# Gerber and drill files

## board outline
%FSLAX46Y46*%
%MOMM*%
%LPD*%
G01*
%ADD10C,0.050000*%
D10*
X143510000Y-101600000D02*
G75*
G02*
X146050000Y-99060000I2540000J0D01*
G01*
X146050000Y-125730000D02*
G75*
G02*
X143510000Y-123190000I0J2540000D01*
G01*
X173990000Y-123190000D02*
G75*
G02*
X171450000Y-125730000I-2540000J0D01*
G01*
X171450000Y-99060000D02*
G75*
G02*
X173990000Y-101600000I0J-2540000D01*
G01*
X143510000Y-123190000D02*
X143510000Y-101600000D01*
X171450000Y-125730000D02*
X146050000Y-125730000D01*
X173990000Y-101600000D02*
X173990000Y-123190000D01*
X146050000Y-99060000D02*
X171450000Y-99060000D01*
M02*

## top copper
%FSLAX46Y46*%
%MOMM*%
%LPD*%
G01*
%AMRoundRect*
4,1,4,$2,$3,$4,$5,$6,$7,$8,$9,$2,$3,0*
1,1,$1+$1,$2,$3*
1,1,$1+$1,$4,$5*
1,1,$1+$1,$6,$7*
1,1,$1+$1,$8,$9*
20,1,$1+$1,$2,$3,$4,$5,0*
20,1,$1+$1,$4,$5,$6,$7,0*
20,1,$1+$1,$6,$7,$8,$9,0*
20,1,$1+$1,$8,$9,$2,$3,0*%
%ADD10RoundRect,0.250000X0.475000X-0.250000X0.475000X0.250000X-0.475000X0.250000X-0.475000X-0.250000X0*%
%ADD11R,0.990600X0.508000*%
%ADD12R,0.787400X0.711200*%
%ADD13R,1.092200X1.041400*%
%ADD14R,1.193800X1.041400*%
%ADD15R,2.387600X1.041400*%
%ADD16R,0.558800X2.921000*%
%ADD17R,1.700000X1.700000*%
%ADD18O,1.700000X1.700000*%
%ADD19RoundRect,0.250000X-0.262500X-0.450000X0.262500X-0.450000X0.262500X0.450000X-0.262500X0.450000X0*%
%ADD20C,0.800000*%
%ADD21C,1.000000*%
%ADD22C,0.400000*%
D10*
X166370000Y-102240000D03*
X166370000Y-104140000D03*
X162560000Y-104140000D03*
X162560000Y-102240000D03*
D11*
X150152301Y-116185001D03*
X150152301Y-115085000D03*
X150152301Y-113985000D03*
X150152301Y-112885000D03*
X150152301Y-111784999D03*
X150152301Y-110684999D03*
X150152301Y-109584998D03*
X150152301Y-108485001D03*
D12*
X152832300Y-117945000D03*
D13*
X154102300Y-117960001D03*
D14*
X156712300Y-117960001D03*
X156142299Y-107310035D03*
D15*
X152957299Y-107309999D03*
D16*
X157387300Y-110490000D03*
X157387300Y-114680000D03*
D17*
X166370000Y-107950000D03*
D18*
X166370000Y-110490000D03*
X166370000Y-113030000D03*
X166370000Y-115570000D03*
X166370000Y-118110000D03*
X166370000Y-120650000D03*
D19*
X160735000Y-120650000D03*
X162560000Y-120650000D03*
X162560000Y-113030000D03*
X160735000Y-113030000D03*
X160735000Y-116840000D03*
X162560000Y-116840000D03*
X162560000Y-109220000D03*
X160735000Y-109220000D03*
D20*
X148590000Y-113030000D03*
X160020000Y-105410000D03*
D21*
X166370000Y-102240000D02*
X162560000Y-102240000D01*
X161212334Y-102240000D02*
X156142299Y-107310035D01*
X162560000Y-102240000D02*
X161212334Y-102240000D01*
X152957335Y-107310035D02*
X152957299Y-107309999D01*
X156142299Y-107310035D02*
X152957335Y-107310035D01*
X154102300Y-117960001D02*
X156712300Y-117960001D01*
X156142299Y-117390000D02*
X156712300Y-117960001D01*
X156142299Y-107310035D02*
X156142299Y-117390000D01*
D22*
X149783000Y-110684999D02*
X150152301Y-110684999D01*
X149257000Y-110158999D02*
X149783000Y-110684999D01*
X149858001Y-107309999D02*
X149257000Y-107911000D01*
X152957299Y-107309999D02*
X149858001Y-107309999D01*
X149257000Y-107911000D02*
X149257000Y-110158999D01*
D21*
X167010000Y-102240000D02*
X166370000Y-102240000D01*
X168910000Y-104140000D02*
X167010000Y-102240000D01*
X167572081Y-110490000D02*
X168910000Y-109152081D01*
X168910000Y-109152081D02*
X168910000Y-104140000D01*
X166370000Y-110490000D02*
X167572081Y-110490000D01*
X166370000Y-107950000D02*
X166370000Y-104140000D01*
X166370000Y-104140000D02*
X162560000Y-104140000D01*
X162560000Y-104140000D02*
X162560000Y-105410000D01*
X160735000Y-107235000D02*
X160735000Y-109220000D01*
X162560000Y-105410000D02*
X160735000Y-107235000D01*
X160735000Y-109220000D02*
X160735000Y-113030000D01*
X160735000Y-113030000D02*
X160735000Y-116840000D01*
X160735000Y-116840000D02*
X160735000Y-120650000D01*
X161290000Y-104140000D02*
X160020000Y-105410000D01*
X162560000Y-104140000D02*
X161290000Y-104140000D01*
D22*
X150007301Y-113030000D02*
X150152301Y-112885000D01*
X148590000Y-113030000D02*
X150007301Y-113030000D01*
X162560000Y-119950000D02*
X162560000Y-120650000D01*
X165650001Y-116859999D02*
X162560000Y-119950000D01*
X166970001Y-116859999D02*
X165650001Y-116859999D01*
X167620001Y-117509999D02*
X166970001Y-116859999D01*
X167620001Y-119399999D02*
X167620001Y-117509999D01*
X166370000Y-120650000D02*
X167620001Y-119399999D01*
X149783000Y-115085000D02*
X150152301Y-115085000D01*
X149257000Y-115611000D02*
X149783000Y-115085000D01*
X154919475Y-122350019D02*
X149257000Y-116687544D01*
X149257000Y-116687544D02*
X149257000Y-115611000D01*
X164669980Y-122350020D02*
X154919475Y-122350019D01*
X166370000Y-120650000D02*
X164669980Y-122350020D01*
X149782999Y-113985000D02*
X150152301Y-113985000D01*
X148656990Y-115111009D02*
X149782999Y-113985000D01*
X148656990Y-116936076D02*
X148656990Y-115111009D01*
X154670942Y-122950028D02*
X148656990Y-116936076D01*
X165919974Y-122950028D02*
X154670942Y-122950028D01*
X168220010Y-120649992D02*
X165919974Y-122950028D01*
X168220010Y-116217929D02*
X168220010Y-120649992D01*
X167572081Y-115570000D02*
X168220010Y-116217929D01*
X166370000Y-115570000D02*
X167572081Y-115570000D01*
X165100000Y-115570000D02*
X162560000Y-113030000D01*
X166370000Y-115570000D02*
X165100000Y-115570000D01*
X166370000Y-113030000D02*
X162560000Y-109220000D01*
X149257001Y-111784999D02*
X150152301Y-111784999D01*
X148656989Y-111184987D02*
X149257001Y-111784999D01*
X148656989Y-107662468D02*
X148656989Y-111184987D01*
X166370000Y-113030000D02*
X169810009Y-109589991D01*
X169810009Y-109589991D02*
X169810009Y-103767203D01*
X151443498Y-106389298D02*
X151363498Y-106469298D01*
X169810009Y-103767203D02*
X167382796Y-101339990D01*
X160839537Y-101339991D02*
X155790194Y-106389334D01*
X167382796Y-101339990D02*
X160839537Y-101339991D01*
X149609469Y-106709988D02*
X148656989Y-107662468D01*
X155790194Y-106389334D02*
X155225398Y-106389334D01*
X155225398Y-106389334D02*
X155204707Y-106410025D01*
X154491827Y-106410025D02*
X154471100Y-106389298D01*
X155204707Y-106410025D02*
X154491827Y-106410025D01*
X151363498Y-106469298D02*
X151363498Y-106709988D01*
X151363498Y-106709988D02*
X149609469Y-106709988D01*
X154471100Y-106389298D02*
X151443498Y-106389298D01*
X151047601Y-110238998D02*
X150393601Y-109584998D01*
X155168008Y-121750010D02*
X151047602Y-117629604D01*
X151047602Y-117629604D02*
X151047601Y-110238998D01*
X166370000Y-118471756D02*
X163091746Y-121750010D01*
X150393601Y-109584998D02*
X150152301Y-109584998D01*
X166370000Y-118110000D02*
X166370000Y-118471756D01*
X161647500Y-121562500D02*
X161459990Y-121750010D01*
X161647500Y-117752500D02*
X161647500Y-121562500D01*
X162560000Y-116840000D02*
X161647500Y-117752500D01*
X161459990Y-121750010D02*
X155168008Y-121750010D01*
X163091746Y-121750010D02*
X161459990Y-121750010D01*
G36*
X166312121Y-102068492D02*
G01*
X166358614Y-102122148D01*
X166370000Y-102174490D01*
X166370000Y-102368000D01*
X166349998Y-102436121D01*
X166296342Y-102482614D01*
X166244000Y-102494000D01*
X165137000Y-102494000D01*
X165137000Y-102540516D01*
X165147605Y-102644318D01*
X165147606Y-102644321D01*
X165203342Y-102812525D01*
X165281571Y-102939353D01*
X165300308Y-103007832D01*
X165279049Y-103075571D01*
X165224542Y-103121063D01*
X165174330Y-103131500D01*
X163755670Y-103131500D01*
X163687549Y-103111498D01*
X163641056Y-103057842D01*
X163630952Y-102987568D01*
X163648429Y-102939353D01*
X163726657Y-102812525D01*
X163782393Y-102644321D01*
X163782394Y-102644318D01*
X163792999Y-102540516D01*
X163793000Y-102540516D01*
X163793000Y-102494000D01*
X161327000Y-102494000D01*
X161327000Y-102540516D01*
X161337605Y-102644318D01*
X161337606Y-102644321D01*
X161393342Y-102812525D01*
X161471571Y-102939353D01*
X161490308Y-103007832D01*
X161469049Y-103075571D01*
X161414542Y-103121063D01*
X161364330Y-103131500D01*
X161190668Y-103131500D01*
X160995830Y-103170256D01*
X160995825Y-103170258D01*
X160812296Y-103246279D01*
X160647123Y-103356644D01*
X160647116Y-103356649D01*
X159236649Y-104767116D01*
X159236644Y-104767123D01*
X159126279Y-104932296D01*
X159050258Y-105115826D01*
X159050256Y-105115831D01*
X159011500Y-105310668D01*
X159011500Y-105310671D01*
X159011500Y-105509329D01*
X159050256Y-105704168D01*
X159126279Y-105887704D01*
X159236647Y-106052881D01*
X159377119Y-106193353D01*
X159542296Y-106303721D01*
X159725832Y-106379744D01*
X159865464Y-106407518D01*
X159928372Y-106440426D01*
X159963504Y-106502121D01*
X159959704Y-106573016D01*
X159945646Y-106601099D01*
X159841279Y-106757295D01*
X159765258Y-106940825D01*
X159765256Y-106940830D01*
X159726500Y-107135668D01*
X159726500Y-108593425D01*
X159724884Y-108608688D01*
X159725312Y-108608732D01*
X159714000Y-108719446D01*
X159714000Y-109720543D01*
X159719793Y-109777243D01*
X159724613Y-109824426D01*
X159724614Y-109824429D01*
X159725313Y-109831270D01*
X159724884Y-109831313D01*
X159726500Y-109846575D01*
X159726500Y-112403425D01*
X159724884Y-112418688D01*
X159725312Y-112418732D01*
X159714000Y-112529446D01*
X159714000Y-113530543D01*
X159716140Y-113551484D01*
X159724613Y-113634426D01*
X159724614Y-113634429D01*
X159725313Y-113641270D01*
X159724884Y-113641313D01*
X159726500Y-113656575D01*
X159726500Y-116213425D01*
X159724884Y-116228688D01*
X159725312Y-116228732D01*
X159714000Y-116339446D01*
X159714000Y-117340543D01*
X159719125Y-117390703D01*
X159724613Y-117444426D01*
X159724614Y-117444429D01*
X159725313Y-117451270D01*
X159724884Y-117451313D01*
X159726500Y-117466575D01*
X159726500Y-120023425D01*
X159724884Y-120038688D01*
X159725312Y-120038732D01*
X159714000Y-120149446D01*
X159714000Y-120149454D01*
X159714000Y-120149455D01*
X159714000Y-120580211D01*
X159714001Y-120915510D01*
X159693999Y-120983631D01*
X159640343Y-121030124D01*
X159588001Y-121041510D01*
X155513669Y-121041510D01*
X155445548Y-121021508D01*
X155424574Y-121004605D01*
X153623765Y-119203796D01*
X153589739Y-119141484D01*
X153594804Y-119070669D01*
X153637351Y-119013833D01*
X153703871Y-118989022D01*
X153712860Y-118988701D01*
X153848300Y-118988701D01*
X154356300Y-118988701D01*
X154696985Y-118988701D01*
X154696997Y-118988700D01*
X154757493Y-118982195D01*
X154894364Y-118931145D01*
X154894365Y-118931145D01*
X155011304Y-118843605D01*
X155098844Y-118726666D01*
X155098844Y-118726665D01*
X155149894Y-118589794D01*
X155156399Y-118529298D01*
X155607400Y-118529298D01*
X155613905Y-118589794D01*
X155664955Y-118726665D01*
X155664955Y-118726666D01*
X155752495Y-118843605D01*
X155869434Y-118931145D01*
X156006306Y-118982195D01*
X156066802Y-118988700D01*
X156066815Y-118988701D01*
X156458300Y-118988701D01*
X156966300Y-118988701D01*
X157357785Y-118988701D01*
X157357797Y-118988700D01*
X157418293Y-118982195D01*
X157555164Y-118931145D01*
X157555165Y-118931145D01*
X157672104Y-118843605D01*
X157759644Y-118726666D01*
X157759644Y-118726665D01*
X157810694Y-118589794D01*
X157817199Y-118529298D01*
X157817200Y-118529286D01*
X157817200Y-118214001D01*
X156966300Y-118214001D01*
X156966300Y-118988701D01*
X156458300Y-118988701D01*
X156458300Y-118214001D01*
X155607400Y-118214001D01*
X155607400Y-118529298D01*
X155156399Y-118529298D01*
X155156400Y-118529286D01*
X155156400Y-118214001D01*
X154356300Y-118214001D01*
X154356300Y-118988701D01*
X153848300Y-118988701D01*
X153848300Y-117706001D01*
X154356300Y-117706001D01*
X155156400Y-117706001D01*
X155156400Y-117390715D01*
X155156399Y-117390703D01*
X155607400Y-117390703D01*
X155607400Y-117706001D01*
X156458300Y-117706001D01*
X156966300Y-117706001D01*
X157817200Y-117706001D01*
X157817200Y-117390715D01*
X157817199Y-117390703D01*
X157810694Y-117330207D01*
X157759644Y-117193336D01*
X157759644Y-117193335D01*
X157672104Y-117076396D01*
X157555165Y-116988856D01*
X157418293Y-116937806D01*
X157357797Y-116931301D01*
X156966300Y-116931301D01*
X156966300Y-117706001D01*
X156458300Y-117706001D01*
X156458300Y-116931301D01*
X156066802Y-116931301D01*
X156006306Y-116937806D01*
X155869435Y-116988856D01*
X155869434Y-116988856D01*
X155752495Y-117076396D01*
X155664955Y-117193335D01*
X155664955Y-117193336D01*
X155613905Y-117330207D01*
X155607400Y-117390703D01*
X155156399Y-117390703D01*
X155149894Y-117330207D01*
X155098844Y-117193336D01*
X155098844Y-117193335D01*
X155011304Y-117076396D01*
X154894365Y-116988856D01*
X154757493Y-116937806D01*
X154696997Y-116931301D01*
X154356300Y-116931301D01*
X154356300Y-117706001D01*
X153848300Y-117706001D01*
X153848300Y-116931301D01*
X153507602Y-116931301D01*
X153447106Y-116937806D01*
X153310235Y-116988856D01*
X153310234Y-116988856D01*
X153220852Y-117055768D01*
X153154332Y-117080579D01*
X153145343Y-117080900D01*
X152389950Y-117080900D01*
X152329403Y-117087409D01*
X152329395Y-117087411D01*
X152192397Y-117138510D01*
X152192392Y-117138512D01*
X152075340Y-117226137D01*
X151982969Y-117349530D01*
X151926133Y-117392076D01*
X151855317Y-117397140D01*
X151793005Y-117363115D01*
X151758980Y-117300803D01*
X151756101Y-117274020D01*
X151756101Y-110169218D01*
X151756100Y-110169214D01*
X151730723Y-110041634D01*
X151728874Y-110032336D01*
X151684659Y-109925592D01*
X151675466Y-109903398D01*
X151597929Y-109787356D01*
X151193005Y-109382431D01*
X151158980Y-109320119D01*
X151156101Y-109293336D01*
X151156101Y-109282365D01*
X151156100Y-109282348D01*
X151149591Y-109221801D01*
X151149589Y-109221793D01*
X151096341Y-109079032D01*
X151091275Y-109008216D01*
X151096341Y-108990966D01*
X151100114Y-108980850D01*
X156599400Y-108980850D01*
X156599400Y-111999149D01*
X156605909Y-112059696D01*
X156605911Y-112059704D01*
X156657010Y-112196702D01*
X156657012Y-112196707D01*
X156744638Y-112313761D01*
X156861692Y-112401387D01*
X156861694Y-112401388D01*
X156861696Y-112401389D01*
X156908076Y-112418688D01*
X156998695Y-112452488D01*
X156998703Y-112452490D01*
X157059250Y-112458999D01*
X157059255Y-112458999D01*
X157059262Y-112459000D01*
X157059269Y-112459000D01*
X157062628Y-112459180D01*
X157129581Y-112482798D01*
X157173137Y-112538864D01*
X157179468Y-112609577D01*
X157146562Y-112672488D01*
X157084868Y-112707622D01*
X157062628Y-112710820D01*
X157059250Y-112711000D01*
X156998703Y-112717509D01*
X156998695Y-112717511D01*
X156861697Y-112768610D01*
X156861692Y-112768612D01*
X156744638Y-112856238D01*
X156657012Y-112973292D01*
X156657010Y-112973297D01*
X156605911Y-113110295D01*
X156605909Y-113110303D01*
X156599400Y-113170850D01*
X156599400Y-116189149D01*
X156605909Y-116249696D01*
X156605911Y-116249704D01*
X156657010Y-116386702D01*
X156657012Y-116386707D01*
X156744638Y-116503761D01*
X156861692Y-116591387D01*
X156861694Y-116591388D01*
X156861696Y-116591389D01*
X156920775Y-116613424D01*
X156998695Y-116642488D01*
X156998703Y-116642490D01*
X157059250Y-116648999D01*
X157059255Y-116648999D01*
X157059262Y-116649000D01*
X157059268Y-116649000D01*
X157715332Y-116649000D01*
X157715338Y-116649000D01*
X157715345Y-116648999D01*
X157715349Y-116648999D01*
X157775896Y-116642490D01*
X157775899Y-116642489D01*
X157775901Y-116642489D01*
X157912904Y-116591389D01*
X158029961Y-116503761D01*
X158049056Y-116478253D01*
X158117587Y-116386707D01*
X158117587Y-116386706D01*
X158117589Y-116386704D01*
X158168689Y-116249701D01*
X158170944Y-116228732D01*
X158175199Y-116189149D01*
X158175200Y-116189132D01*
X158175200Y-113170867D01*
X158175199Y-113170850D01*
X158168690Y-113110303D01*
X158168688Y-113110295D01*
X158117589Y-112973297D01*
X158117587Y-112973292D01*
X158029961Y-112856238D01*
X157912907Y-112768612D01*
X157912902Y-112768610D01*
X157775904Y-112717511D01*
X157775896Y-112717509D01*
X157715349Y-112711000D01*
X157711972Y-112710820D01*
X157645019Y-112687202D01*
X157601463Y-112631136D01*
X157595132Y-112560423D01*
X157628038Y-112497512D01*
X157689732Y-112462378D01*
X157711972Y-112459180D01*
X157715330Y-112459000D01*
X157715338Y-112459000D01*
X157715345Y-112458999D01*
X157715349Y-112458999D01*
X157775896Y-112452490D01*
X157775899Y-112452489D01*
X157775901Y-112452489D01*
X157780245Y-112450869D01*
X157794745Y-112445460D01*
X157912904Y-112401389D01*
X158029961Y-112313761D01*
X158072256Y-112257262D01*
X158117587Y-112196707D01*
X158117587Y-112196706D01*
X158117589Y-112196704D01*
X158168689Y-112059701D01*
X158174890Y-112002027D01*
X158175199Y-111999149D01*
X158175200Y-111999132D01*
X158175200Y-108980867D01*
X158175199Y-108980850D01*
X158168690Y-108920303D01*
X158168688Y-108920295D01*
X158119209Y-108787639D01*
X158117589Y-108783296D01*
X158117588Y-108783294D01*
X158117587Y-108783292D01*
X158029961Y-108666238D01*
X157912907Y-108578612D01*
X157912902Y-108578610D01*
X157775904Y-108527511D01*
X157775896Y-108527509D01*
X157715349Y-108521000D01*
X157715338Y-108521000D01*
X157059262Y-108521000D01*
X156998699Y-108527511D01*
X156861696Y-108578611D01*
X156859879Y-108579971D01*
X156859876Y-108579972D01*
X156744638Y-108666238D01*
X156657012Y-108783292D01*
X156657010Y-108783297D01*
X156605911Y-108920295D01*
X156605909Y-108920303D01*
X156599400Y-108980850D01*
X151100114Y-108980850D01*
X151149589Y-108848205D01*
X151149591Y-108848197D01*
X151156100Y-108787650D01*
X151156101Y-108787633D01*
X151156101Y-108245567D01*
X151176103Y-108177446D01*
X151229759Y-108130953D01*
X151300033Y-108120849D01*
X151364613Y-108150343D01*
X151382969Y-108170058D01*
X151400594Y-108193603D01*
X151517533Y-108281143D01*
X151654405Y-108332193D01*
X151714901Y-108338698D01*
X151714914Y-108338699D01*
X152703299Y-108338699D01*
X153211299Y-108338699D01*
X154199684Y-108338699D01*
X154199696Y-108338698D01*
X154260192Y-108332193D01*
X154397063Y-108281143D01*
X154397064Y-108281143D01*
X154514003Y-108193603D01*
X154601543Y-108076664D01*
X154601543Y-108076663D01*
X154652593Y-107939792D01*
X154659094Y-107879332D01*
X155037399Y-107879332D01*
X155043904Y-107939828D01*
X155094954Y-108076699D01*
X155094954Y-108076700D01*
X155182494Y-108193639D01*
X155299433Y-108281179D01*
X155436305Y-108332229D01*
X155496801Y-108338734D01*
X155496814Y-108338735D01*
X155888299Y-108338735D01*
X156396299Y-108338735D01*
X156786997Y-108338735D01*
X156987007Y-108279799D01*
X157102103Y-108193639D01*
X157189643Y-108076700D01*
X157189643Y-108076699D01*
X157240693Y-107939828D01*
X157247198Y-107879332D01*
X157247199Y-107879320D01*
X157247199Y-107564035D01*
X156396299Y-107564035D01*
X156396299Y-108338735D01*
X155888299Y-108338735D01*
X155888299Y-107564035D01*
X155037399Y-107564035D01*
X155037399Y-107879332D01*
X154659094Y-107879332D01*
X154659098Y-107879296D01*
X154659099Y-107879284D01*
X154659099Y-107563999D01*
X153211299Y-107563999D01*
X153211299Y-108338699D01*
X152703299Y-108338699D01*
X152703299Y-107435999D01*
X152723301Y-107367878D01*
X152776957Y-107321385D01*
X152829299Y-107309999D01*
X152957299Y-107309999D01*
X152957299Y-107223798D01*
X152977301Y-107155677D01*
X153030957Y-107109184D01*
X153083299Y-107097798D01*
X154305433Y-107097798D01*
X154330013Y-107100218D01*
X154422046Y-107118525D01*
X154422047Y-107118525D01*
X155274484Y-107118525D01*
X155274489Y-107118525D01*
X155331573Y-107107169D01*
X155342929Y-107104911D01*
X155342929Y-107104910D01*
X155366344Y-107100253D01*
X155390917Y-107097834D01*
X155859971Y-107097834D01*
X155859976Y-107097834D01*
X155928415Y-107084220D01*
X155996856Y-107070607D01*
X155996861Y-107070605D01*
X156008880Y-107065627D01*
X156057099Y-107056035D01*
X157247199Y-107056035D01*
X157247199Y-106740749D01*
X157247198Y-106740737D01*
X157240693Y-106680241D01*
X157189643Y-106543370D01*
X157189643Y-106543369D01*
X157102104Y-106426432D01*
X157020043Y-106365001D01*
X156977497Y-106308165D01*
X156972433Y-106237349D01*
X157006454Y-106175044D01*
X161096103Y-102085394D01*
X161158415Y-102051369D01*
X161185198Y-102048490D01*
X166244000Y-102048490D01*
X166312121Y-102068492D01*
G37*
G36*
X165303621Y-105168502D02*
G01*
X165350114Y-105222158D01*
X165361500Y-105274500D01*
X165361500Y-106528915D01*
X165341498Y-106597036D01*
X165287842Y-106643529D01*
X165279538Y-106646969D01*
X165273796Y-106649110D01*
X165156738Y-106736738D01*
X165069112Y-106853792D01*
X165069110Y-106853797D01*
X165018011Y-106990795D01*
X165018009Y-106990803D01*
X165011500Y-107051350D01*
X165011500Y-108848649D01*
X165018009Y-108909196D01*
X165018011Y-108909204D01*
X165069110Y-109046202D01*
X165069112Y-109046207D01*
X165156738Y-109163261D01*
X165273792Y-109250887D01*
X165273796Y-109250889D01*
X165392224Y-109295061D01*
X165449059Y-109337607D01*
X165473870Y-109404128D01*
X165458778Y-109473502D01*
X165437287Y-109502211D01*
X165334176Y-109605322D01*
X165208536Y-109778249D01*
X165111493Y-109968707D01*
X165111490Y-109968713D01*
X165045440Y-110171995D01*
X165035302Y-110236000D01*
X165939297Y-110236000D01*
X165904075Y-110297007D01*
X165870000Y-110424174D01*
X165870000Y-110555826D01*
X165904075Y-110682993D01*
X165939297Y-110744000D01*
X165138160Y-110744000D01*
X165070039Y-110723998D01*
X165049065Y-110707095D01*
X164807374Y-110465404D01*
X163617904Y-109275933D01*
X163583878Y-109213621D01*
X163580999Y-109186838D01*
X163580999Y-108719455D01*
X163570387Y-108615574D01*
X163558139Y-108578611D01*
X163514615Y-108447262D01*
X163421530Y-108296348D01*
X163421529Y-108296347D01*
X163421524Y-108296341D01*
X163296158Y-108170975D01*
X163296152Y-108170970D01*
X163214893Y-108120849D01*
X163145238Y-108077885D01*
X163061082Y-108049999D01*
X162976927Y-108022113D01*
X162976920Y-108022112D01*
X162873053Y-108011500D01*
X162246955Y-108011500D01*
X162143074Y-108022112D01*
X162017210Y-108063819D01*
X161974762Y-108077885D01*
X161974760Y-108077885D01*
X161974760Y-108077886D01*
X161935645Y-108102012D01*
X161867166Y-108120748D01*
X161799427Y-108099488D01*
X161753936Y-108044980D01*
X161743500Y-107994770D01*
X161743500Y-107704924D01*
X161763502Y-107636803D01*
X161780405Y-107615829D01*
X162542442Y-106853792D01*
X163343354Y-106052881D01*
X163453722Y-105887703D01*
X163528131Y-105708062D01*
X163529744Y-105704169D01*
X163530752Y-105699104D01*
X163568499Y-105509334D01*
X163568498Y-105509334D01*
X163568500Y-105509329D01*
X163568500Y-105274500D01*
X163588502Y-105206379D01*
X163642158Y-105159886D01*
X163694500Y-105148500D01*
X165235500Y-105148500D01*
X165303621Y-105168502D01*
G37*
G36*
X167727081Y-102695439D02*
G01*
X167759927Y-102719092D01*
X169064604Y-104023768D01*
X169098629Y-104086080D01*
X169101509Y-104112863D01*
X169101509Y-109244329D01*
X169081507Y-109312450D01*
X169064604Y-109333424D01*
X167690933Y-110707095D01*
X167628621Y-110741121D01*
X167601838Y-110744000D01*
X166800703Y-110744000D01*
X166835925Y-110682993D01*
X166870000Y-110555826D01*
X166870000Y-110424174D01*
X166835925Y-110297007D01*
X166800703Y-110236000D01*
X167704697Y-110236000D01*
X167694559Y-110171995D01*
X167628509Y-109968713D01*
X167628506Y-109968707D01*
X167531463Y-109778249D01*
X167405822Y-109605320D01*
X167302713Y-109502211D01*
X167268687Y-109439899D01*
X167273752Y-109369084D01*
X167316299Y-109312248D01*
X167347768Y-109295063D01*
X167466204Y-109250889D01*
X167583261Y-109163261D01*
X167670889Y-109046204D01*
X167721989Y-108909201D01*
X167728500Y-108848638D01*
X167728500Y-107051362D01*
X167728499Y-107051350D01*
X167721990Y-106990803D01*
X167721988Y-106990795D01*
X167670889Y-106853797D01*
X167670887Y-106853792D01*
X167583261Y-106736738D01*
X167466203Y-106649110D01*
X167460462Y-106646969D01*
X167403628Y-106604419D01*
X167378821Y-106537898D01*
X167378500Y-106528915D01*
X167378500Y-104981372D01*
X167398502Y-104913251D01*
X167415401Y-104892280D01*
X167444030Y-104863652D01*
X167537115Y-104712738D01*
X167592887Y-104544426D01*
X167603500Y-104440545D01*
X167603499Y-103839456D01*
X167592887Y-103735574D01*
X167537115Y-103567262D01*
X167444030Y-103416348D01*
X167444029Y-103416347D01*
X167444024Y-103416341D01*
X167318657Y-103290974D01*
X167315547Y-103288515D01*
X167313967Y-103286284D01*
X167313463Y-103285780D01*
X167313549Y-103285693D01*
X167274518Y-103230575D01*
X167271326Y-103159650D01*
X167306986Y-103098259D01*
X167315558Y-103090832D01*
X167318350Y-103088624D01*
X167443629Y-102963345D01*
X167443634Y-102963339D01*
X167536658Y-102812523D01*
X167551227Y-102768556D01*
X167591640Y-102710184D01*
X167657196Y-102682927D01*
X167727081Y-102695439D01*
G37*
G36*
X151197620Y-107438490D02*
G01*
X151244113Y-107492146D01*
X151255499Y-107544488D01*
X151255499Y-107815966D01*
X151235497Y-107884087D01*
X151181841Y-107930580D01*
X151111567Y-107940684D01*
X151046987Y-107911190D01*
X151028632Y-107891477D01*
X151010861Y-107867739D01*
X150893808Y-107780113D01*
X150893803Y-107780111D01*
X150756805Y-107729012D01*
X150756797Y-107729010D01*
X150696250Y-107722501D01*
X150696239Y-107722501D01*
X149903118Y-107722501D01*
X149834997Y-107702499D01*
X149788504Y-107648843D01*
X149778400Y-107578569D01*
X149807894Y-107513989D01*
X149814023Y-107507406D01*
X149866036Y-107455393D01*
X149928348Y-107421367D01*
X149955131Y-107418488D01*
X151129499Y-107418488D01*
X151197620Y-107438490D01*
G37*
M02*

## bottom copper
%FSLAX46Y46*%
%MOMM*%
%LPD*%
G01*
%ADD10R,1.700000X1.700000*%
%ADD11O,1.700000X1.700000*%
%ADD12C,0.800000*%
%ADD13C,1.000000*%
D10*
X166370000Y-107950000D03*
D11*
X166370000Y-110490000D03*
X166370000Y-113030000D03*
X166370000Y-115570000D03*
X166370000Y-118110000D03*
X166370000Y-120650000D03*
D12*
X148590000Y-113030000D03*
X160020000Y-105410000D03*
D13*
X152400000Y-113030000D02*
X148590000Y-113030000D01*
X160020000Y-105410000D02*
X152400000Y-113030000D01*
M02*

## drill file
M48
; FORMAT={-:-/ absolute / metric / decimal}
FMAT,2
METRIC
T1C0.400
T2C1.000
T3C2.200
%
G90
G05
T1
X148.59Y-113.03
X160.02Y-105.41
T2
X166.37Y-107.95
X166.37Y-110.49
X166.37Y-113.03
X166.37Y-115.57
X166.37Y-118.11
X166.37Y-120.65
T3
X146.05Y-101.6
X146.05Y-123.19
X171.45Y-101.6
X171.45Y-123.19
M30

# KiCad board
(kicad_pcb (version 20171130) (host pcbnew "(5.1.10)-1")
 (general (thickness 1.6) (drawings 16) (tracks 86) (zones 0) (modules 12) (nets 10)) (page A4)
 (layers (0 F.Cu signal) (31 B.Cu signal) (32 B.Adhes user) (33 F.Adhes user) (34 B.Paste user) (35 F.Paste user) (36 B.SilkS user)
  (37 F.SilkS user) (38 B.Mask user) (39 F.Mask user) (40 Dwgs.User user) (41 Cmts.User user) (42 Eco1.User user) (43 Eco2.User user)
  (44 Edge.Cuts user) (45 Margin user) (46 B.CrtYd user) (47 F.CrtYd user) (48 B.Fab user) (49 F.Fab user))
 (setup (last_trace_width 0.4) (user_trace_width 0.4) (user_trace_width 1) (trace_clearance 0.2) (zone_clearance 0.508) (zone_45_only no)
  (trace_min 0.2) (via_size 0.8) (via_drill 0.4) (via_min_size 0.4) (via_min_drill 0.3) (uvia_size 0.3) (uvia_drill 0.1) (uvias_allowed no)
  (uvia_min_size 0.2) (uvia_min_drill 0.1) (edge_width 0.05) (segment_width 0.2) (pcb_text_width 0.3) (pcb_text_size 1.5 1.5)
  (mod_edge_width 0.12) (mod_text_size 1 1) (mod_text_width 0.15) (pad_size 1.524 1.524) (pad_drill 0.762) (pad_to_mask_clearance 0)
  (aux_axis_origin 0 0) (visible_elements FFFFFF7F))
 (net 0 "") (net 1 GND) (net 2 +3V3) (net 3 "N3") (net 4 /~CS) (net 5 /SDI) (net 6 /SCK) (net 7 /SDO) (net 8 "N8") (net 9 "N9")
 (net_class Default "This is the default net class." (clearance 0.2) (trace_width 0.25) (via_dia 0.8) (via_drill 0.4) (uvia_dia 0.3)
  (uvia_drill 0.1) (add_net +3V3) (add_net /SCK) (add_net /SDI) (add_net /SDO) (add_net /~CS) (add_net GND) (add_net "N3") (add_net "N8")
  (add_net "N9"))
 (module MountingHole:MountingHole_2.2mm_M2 (layer F.Cu) (at 171.45 123.19)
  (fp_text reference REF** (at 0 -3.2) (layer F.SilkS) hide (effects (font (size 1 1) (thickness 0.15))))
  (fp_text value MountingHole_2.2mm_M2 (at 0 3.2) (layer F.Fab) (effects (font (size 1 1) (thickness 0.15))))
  (pad 1 np_thru_hole circle (at 0 0) (size 2.2 2.2) (drill 2.2) (layers *.Cu *.Mask)))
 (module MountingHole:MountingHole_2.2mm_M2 (layer F.Cu) (at 146.05 123.19)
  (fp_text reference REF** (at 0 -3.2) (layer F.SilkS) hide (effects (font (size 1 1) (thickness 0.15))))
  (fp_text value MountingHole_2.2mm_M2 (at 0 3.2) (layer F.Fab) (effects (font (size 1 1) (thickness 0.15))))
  (pad 1 np_thru_hole circle (at 0 0) (size 2.2 2.2) (drill 2.2) (layers *.Cu *.Mask)))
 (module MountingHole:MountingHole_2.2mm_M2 (layer F.Cu) (at 146.05 101.6)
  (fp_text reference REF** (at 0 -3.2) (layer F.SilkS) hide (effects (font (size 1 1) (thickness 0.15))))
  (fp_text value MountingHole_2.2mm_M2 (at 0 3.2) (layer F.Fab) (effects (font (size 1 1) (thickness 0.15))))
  (pad 1 np_thru_hole circle (at 0 0) (size 2.2 2.2) (drill 2.2) (layers *.Cu *.Mask)))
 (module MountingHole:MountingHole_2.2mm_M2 (layer F.Cu) (at 171.45 101.6)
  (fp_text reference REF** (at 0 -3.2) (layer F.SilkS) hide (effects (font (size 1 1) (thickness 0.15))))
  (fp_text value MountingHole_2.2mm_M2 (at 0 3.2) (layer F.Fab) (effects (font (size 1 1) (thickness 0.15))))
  (pad 1 np_thru_hole circle (at 0 0) (size 2.2 2.2) (drill 2.2) (layers *.Cu *.Mask)))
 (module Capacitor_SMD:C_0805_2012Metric (layer F.Cu) (at 166.37 103.19 90)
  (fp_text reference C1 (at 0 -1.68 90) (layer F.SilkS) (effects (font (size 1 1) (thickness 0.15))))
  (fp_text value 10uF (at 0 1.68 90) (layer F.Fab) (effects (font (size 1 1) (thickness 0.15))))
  (pad 2 smd roundrect (at 0.95 0 90) (size 1 1.45) (layers F.Cu F.Paste F.Mask) (roundrect_rratio 0.25) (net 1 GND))
  (pad 1 smd roundrect (at -0.95 0 90) (size 1 1.45) (layers F.Cu F.Paste F.Mask) (roundrect_rratio 0.25) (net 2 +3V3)))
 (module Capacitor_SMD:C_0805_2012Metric (layer F.Cu) (at 162.56 103.19 90)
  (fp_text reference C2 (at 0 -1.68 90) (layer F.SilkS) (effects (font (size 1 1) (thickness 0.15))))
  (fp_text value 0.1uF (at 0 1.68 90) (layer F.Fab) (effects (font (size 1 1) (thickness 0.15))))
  (pad 1 smd roundrect (at -0.95 0 90) (size 1 1.45) (layers F.Cu F.Paste F.Mask) (roundrect_rratio 0.25) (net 2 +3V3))
  (pad 2 smd roundrect (at 0.95 0 90) (size 1 1.45) (layers F.Cu F.Paste F.Mask) (roundrect_rratio 0.25) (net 1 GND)))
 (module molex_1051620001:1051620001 (layer F.Cu) (at 153.67 112.635 270)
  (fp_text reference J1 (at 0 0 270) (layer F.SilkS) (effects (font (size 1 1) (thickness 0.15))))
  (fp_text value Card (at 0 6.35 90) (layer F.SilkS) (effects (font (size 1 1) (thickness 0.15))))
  (pad P1 smd rect (at 3.550001 3.517699 270) (size 0.508 0.9906) (layers F.Cu F.Paste F.Mask) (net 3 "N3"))
  (pad P2 smd rect (at 2.45 3.517699 270) (size 0.508 0.9906) (layers F.Cu F.Paste F.Mask) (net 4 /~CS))
  (pad P3 smd rect (at 1.35 3.517699 270) (size 0.508 0.9906) (layers F.Cu F.Paste F.Mask) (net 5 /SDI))
  (pad P4 smd rect (at 0.25 3.517699 270) (size 0.508 0.9906) (layers F.Cu F.Paste F.Mask) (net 2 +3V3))
  (pad P5 smd rect (at -0.850001 3.517699 270) (size 0.508 0.9906) (layers F.Cu F.Paste F.Mask) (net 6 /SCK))
  (pad P6 smd rect (at -1.950001 3.517699 270) (size 0.508 0.9906) (layers F.Cu F.Paste F.Mask) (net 1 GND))
  (pad P7 smd rect (at -3.050002 3.517699 270) (size 0.508 0.9906) (layers F.Cu F.Paste F.Mask) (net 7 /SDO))
  (pad P8 smd rect (at -4.149999 3.517699 270) (size 0.508 0.9906) (layers F.Cu F.Paste F.Mask) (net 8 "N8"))
  (pad P9 smd rect (at 5.31 0.8377 270) (size 0.7112 0.7874) (layers F.Cu F.Paste F.Mask) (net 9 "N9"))
  (pad G1 smd rect (at 5.325001 -0.4323 270) (size 1.0414 1.0922) (layers F.Cu F.Paste F.Mask) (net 1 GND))
  (pad G2 smd rect (at 5.325001 -3.0423 270) (size 1.0414 1.1938) (layers F.Cu F.Paste F.Mask) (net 1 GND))
  (pad G3 smd rect (at -5.324965 -2.472299 270) (size 1.0414 1.1938) (layers F.Cu F.Paste F.Mask) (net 1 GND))
  (pad G4 smd rect (at -5.325001 0.712701 270) (size 1.0414 2.3876) (layers F.Cu F.Paste F.Mask) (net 1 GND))
  (pad 14 smd rect (at -2.145 -3.7173 270) (size 2.921 0.5588) (layers F.Cu F.Paste F.Mask))
  (pad 15 smd rect (at 2.045 -3.7173 270) (size 2.921 0.5588) (layers F.Cu F.Paste F.Mask)))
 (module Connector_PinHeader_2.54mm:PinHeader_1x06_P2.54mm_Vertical (layer F.Cu) (at 166.37 107.95)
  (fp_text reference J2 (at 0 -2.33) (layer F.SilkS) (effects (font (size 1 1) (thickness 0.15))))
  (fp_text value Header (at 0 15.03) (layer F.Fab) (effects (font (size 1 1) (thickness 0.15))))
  (pad 1 thru_hole rect (at 0 0) (size 1.7 1.7) (drill 1) (layers *.Cu *.Mask) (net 2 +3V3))
  (pad 2 thru_hole oval (at 0 2.54) (size 1.7 1.7) (drill 1) (layers *.Cu *.Mask) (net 1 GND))
  (pad 3 thru_hole oval (at 0 5.08) (size 1.7 1.7) (drill 1) (layers *.Cu *.Mask) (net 6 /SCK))
  (pad 4 thru_hole oval (at 0 7.62) (size 1.7 1.7) (drill 1) (layers *.Cu *.Mask) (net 5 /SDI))
  (pad 5 thru_hole oval (at 0 10.16) (size 1.7 1.7) (drill 1) (layers *.Cu *.Mask) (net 7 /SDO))
  (pad 6 thru_hole oval (at 0 12.7) (size 1.7 1.7) (drill 1) (layers *.Cu *.Mask) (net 4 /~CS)))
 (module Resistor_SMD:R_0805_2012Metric (layer F.Cu) (at 161.6475 120.65)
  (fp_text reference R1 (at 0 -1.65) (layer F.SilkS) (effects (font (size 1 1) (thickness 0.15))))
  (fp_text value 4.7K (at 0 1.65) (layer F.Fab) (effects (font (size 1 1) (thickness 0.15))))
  (pad 1 smd roundrect (at -0.9125 0) (size 1.025 1.4) (layers F.Cu F.Paste F.Mask) (roundrect_rratio 0.243902) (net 2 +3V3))
  (pad 2 smd roundrect (at 0.9125 0) (size 1.025 1.4) (layers F.Cu F.Paste F.Mask) (roundrect_rratio 0.243902) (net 4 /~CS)))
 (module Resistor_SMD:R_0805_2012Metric (layer F.Cu) (at 161.6475 113.03)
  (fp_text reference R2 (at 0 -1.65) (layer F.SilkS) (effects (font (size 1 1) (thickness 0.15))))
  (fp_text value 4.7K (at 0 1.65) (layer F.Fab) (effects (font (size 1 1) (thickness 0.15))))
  (pad 2 smd roundrect (at 0.9125 0) (size 1.025 1.4) (layers F.Cu F.Paste F.Mask) (roundrect_rratio 0.243902) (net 5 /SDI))
  (pad 1 smd roundrect (at -0.9125 0) (size 1.025 1.4) (layers F.Cu F.Paste F.Mask) (roundrect_rratio 0.243902) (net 2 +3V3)))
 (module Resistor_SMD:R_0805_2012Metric (layer F.Cu) (at 161.6475 116.84)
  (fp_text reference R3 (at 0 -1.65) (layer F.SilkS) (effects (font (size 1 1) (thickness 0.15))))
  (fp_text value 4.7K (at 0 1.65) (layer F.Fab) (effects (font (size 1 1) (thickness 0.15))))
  (pad 1 smd roundrect (at -0.9125 0) (size 1.025 1.4) (layers F.Cu F.Paste F.Mask) (roundrect_rratio 0.243902) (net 2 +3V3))
  (pad 2 smd roundrect (at 0.9125 0) (size 1.025 1.4) (layers F.Cu F.Paste F.Mask) (roundrect_rratio 0.243902) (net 7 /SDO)))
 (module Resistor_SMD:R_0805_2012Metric (layer F.Cu) (at 161.6475 109.22)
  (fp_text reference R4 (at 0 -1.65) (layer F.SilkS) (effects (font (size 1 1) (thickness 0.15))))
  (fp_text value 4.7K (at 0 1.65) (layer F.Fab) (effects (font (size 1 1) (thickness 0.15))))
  (pad 2 smd roundrect (at 0.9125 0) (size 1.025 1.4) (layers F.Cu F.Paste F.Mask) (roundrect_rratio 0.243902) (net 6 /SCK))
  (pad 1 smd roundrect (at -0.9125 0) (size 1.025 1.4) (layers F.Cu F.Paste F.Mask) (roundrect_rratio 0.243902) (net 2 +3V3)))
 (gr_arc (start 146.05 101.6) (end 146.05 99.06) (angle -90) (layer Edge.Cuts) (width 0.05))
 (gr_arc (start 146.05 123.19) (end 143.51 123.19) (angle -90) (layer Edge.Cuts) (width 0.05))
 (gr_arc (start 171.45 123.19) (end 171.45 125.73) (angle -90) (layer Edge.Cuts) (width 0.05))
 (gr_arc (start 171.45 101.6) (end 173.99 101.6) (angle -90) (layer Edge.Cuts) (width 0.05))
 (gr_line (start 143.51 123.19) (end 143.51 101.6) (layer Edge.Cuts) (width 0.05))
 (gr_line (start 171.45 125.73) (end 146.05 125.73) (layer Edge.Cuts) (width 0.05))
 (gr_line (start 173.99 101.6) (end 173.99 123.19) (layer Edge.Cuts) (width 0.05))
 (gr_line (start 146.05 99.06) (end 171.45 99.06) (layer Edge.Cuts) (width 0.05))
 (segment (start 166.37 102.24) (end 162.56 102.24) (width 1) (layer F.Cu) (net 1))
 (segment (start 161.212334 102.24) (end 156.142299 107.310035) (width 1) (layer F.Cu) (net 1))
 (segment (start 162.56 102.24) (end 161.212334 102.24) (width 1) (layer F.Cu) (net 1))
 (segment (start 152.957335 107.310035) (end 152.957299 107.309999) (width 1) (layer F.Cu) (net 1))
 (segment (start 156.142299 107.310035) (end 152.957335 107.310035) (width 1) (layer F.Cu) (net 1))
 (segment (start 154.1023 117.960001) (end 156.7123 117.960001) (width 1) (layer F.Cu) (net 1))
 (segment (start 156.142299 117.39) (end 156.7123 117.960001) (width 1) (layer F.Cu) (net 1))
 (segment (start 156.142299 107.310035) (end 156.142299 117.39) (width 1) (layer F.Cu) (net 1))
 (segment (start 149.783 110.684999) (end 150.152301 110.684999) (width 0.4) (layer F.Cu) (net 1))
 (segment (start 149.257 110.158999) (end 149.783 110.684999) (width 0.4) (layer F.Cu) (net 1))
 (segment (start 149.858001 107.309999) (end 149.257 107.911) (width 0.4) (layer F.Cu) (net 1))
 (segment (start 152.957299 107.309999) (end 149.858001 107.309999) (width 0.4) (layer F.Cu) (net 1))
 (segment (start 149.257 107.911) (end 149.257 110.158999) (width 0.4) (layer F.Cu) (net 1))
 (segment (start 167.01 102.24) (end 166.37 102.24) (width 1) (layer F.Cu) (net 1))
 (segment (start 168.91 104.14) (end 167.01 102.24) (width 1) (layer F.Cu) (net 1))
 (segment (start 167.572081 110.49) (end 168.91 109.152081) (width 1) (layer F.Cu) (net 1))
 (segment (start 168.91 109.152081) (end 168.91 104.14) (width 1) (layer F.Cu) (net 1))
 (segment (start 166.37 110.49) (end 167.572081 110.49) (width 1) (layer F.Cu) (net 1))
 (segment (start 166.37 107.95) (end 166.37 104.14) (width 1) (layer F.Cu) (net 2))
 (segment (start 166.37 104.14) (end 162.56 104.14) (width 1) (layer F.Cu) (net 2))
 (segment (start 162.56 104.14) (end 162.56 105.41) (width 1) (layer F.Cu) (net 2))
 (segment (start 160.735 107.235) (end 160.735 109.22) (width 1) (layer F.Cu) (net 2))
 (segment (start 162.56 105.41) (end 160.735 107.235) (width 1) (layer F.Cu) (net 2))
 (segment (start 160.735 109.22) (end 160.735 113.03) (width 1) (layer F.Cu) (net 2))
 (segment (start 160.735 113.03) (end 160.735 116.84) (width 1) (layer F.Cu) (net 2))
 (segment (start 160.735 116.84) (end 160.735 120.65) (width 1) (layer F.Cu) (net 2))
 (via (at 148.59 113.03) (size 0.8) (drill 0.4) (layers F.Cu B.Cu) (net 2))
 (via (at 160.02 105.41) (size 0.8) (drill 0.4) (layers F.Cu B.Cu) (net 2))
 (segment (start 161.29 104.14) (end 160.02 105.41) (width 1) (layer F.Cu) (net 2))
 (segment (start 162.56 104.14) (end 161.29 104.14) (width 1) (layer F.Cu) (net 2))
 (segment (start 152.4 113.03) (end 148.59 113.03) (width 1) (layer B.Cu) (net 2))
 (segment (start 160.02 105.41) (end 152.4 113.03) (width 1) (layer B.Cu) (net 2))
 (segment (start 150.007301 113.03) (end 150.152301 112.885) (width 0.4) (layer F.Cu) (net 2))
 (segment (start 148.59 113.03) (end 150.007301 113.03) (width 0.4) (layer F.Cu) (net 2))
 (segment (start 162.56 119.95) (end 162.56 120.65) (width 0.4) (layer F.Cu) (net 4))
 (segment (start 165.650001 116.859999) (end 162.56 119.95) (width 0.4) (layer F.Cu) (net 4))
 (segment (start 166.970001 116.859999) (end 165.650001 116.859999) (width 0.4) (layer F.Cu) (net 4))
 (segment (start 167.620001 117.509999) (end 166.970001 116.859999) (width 0.4) (layer F.Cu) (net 4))
 (segment (start 167.620001 119.399999) (end 167.620001 117.509999) (width 0.4) (layer F.Cu) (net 4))
 (segment (start 166.37 120.65) (end 167.620001 119.399999) (width 0.4) (layer F.Cu) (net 4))
 (segment (start 149.783 115.085) (end 150.152301 115.085) (width 0.4) (layer F.Cu) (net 4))
 (segment (start 149.257 115.611) (end 149.783 115.085) (width 0.4) (layer F.Cu) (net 4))
 (segment (start 154.919475 122.350019) (end 149.257 116.687544) (width 0.4) (layer F.Cu) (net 4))
 (segment (start 149.257 116.687544) (end 149.257 115.611) (width 0.4) (layer F.Cu) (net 4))
 (segment (start 164.66998 122.35002) (end 154.919475 122.350019) (width 0.4) (layer F.Cu) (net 4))
 (segment (start 166.37 120.65) (end 164.66998 122.35002) (width 0.4) (layer F.Cu) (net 4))
 (segment (start 149.782999 113.985) (end 150.152301 113.985) (width 0.4) (layer F.Cu) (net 5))
 (segment (start 148.65699 115.111009) (end 149.782999 113.985) (width 0.4) (layer F.Cu) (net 5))
 (segment (start 148.65699 116.936076) (end 148.65699 115.111009) (width 0.4) (layer F.Cu) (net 5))
 (segment (start 154.670942 122.950028) (end 148.65699 116.936076) (width 0.4) (layer F.Cu) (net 5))
 (segment (start 165.919974 122.950028) (end 154.670942 122.950028) (width 0.4) (layer F.Cu) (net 5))
 (segment (start 168.22001 120.649992) (end 165.919974 122.950028) (width 0.4) (layer F.Cu) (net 5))
 (segment (start 168.22001 116.217929) (end 168.22001 120.649992) (width 0.4) (layer F.Cu) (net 5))
 (segment (start 167.572081 115.57) (end 168.22001 116.217929) (width 0.4) (layer F.Cu) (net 5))
 (segment (start 166.37 115.57) (end 167.572081 115.57) (width 0.4) (layer F.Cu) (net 5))
 (segment (start 165.1 115.57) (end 162.56 113.03) (width 0.4) (layer F.Cu) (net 5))
 (segment (start 166.37 115.57) (end 165.1 115.57) (width 0.4) (layer F.Cu) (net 5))
 (segment (start 166.37 113.03) (end 162.56 109.22) (width 0.4) (layer F.Cu) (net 6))
 (segment (start 149.257001 111.784999) (end 150.152301 111.784999) (width 0.4) (layer F.Cu) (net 6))
 (segment (start 148.656989 111.184987) (end 149.257001 111.784999) (width 0.4) (layer F.Cu) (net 6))
 (segment (start 148.656989 107.662468) (end 148.656989 111.184987) (width 0.4) (layer F.Cu) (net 6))
 (segment (start 166.37 113.03) (end 169.810009 109.589991) (width 0.4) (layer F.Cu) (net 6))
 (segment (start 169.810009 109.589991) (end 169.810009 103.767203) (width 0.4) (layer F.Cu) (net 6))
 (segment (start 151.443498 106.389298) (end 151.363498 106.469298) (width 0.4) (layer F.Cu) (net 6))
 (segment (start 169.810009 103.767203) (end 167.382796 101.33999) (width 0.4) (layer F.Cu) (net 6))
 (segment (start 160.839537 101.339991) (end 155.790194 106.389334) (width 0.4) (layer F.Cu) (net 6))
 (segment (start 167.382796 101.33999) (end 160.839537 101.339991) (width 0.4) (layer F.Cu) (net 6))
 (segment (start 149.609469 106.709988) (end 148.656989 107.662468) (width 0.4) (layer F.Cu) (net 6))
 (segment (start 155.790194 106.389334) (end 155.225398 106.389334) (width 0.4) (layer F.Cu) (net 6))
 (segment (start 155.225398 106.389334) (end 155.204707 106.410025) (width 0.4) (layer F.Cu) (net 6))
 (segment (start 154.491827 106.410025) (end 154.4711 106.389298) (width 0.4) (layer F.Cu) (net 6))
 (segment (start 155.204707 106.410025) (end 154.491827 106.410025) (width 0.4) (layer F.Cu) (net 6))
 (segment (start 151.363498 106.469298) (end 151.363498 106.709988) (width 0.4) (layer F.Cu) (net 6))
 (segment (start 151.363498 106.709988) (end 149.609469 106.709988) (width 0.4) (layer F.Cu) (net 6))
 (segment (start 154.4711 106.389298) (end 151.443498 106.389298) (width 0.4) (layer F.Cu) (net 6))
 (segment (start 151.047601 110.238998) (end 150.393601 109.584998) (width 0.4) (layer F.Cu) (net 7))
 (segment (start 155.168008 121.75001) (end 151.047602 117.629604) (width 0.4) (layer F.Cu) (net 7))
 (segment (start 151.047602 117.629604) (end 151.047601 110.238998) (width 0.4) (layer F.Cu) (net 7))
 (segment (start 166.37 118.471756) (end 163.091746 121.75001) (width 0.4) (layer F.Cu) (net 7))
 (segment (start 150.393601 109.584998) (end 150.152301 109.584998) (width 0.4) (layer F.Cu) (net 7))
 (segment (start 166.37 118.11) (end 166.37 118.471756) (width 0.4) (layer F.Cu) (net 7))
 (segment (start 161.6475 121.5625) (end 161.45999 121.75001) (width 0.4) (layer F.Cu) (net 7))
 (segment (start 161.6475 117.7525) (end 161.6475 121.5625) (width 0.4) (layer F.Cu) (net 7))
 (segment (start 162.56 116.84) (end 161.6475 117.7525) (width 0.4) (layer F.Cu) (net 7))
 (segment (start 161.45999 121.75001) (end 155.168008 121.75001) (width 0.4) (layer F.Cu) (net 7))
 (segment (start 163.091746 121.75001) (end 161.45999 121.75001) (width 0.4) (layer F.Cu) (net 7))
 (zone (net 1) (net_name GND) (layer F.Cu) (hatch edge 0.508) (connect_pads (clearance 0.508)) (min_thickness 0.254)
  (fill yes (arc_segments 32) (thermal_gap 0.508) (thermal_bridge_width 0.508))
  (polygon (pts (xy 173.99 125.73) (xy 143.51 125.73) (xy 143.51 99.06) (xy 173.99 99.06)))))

